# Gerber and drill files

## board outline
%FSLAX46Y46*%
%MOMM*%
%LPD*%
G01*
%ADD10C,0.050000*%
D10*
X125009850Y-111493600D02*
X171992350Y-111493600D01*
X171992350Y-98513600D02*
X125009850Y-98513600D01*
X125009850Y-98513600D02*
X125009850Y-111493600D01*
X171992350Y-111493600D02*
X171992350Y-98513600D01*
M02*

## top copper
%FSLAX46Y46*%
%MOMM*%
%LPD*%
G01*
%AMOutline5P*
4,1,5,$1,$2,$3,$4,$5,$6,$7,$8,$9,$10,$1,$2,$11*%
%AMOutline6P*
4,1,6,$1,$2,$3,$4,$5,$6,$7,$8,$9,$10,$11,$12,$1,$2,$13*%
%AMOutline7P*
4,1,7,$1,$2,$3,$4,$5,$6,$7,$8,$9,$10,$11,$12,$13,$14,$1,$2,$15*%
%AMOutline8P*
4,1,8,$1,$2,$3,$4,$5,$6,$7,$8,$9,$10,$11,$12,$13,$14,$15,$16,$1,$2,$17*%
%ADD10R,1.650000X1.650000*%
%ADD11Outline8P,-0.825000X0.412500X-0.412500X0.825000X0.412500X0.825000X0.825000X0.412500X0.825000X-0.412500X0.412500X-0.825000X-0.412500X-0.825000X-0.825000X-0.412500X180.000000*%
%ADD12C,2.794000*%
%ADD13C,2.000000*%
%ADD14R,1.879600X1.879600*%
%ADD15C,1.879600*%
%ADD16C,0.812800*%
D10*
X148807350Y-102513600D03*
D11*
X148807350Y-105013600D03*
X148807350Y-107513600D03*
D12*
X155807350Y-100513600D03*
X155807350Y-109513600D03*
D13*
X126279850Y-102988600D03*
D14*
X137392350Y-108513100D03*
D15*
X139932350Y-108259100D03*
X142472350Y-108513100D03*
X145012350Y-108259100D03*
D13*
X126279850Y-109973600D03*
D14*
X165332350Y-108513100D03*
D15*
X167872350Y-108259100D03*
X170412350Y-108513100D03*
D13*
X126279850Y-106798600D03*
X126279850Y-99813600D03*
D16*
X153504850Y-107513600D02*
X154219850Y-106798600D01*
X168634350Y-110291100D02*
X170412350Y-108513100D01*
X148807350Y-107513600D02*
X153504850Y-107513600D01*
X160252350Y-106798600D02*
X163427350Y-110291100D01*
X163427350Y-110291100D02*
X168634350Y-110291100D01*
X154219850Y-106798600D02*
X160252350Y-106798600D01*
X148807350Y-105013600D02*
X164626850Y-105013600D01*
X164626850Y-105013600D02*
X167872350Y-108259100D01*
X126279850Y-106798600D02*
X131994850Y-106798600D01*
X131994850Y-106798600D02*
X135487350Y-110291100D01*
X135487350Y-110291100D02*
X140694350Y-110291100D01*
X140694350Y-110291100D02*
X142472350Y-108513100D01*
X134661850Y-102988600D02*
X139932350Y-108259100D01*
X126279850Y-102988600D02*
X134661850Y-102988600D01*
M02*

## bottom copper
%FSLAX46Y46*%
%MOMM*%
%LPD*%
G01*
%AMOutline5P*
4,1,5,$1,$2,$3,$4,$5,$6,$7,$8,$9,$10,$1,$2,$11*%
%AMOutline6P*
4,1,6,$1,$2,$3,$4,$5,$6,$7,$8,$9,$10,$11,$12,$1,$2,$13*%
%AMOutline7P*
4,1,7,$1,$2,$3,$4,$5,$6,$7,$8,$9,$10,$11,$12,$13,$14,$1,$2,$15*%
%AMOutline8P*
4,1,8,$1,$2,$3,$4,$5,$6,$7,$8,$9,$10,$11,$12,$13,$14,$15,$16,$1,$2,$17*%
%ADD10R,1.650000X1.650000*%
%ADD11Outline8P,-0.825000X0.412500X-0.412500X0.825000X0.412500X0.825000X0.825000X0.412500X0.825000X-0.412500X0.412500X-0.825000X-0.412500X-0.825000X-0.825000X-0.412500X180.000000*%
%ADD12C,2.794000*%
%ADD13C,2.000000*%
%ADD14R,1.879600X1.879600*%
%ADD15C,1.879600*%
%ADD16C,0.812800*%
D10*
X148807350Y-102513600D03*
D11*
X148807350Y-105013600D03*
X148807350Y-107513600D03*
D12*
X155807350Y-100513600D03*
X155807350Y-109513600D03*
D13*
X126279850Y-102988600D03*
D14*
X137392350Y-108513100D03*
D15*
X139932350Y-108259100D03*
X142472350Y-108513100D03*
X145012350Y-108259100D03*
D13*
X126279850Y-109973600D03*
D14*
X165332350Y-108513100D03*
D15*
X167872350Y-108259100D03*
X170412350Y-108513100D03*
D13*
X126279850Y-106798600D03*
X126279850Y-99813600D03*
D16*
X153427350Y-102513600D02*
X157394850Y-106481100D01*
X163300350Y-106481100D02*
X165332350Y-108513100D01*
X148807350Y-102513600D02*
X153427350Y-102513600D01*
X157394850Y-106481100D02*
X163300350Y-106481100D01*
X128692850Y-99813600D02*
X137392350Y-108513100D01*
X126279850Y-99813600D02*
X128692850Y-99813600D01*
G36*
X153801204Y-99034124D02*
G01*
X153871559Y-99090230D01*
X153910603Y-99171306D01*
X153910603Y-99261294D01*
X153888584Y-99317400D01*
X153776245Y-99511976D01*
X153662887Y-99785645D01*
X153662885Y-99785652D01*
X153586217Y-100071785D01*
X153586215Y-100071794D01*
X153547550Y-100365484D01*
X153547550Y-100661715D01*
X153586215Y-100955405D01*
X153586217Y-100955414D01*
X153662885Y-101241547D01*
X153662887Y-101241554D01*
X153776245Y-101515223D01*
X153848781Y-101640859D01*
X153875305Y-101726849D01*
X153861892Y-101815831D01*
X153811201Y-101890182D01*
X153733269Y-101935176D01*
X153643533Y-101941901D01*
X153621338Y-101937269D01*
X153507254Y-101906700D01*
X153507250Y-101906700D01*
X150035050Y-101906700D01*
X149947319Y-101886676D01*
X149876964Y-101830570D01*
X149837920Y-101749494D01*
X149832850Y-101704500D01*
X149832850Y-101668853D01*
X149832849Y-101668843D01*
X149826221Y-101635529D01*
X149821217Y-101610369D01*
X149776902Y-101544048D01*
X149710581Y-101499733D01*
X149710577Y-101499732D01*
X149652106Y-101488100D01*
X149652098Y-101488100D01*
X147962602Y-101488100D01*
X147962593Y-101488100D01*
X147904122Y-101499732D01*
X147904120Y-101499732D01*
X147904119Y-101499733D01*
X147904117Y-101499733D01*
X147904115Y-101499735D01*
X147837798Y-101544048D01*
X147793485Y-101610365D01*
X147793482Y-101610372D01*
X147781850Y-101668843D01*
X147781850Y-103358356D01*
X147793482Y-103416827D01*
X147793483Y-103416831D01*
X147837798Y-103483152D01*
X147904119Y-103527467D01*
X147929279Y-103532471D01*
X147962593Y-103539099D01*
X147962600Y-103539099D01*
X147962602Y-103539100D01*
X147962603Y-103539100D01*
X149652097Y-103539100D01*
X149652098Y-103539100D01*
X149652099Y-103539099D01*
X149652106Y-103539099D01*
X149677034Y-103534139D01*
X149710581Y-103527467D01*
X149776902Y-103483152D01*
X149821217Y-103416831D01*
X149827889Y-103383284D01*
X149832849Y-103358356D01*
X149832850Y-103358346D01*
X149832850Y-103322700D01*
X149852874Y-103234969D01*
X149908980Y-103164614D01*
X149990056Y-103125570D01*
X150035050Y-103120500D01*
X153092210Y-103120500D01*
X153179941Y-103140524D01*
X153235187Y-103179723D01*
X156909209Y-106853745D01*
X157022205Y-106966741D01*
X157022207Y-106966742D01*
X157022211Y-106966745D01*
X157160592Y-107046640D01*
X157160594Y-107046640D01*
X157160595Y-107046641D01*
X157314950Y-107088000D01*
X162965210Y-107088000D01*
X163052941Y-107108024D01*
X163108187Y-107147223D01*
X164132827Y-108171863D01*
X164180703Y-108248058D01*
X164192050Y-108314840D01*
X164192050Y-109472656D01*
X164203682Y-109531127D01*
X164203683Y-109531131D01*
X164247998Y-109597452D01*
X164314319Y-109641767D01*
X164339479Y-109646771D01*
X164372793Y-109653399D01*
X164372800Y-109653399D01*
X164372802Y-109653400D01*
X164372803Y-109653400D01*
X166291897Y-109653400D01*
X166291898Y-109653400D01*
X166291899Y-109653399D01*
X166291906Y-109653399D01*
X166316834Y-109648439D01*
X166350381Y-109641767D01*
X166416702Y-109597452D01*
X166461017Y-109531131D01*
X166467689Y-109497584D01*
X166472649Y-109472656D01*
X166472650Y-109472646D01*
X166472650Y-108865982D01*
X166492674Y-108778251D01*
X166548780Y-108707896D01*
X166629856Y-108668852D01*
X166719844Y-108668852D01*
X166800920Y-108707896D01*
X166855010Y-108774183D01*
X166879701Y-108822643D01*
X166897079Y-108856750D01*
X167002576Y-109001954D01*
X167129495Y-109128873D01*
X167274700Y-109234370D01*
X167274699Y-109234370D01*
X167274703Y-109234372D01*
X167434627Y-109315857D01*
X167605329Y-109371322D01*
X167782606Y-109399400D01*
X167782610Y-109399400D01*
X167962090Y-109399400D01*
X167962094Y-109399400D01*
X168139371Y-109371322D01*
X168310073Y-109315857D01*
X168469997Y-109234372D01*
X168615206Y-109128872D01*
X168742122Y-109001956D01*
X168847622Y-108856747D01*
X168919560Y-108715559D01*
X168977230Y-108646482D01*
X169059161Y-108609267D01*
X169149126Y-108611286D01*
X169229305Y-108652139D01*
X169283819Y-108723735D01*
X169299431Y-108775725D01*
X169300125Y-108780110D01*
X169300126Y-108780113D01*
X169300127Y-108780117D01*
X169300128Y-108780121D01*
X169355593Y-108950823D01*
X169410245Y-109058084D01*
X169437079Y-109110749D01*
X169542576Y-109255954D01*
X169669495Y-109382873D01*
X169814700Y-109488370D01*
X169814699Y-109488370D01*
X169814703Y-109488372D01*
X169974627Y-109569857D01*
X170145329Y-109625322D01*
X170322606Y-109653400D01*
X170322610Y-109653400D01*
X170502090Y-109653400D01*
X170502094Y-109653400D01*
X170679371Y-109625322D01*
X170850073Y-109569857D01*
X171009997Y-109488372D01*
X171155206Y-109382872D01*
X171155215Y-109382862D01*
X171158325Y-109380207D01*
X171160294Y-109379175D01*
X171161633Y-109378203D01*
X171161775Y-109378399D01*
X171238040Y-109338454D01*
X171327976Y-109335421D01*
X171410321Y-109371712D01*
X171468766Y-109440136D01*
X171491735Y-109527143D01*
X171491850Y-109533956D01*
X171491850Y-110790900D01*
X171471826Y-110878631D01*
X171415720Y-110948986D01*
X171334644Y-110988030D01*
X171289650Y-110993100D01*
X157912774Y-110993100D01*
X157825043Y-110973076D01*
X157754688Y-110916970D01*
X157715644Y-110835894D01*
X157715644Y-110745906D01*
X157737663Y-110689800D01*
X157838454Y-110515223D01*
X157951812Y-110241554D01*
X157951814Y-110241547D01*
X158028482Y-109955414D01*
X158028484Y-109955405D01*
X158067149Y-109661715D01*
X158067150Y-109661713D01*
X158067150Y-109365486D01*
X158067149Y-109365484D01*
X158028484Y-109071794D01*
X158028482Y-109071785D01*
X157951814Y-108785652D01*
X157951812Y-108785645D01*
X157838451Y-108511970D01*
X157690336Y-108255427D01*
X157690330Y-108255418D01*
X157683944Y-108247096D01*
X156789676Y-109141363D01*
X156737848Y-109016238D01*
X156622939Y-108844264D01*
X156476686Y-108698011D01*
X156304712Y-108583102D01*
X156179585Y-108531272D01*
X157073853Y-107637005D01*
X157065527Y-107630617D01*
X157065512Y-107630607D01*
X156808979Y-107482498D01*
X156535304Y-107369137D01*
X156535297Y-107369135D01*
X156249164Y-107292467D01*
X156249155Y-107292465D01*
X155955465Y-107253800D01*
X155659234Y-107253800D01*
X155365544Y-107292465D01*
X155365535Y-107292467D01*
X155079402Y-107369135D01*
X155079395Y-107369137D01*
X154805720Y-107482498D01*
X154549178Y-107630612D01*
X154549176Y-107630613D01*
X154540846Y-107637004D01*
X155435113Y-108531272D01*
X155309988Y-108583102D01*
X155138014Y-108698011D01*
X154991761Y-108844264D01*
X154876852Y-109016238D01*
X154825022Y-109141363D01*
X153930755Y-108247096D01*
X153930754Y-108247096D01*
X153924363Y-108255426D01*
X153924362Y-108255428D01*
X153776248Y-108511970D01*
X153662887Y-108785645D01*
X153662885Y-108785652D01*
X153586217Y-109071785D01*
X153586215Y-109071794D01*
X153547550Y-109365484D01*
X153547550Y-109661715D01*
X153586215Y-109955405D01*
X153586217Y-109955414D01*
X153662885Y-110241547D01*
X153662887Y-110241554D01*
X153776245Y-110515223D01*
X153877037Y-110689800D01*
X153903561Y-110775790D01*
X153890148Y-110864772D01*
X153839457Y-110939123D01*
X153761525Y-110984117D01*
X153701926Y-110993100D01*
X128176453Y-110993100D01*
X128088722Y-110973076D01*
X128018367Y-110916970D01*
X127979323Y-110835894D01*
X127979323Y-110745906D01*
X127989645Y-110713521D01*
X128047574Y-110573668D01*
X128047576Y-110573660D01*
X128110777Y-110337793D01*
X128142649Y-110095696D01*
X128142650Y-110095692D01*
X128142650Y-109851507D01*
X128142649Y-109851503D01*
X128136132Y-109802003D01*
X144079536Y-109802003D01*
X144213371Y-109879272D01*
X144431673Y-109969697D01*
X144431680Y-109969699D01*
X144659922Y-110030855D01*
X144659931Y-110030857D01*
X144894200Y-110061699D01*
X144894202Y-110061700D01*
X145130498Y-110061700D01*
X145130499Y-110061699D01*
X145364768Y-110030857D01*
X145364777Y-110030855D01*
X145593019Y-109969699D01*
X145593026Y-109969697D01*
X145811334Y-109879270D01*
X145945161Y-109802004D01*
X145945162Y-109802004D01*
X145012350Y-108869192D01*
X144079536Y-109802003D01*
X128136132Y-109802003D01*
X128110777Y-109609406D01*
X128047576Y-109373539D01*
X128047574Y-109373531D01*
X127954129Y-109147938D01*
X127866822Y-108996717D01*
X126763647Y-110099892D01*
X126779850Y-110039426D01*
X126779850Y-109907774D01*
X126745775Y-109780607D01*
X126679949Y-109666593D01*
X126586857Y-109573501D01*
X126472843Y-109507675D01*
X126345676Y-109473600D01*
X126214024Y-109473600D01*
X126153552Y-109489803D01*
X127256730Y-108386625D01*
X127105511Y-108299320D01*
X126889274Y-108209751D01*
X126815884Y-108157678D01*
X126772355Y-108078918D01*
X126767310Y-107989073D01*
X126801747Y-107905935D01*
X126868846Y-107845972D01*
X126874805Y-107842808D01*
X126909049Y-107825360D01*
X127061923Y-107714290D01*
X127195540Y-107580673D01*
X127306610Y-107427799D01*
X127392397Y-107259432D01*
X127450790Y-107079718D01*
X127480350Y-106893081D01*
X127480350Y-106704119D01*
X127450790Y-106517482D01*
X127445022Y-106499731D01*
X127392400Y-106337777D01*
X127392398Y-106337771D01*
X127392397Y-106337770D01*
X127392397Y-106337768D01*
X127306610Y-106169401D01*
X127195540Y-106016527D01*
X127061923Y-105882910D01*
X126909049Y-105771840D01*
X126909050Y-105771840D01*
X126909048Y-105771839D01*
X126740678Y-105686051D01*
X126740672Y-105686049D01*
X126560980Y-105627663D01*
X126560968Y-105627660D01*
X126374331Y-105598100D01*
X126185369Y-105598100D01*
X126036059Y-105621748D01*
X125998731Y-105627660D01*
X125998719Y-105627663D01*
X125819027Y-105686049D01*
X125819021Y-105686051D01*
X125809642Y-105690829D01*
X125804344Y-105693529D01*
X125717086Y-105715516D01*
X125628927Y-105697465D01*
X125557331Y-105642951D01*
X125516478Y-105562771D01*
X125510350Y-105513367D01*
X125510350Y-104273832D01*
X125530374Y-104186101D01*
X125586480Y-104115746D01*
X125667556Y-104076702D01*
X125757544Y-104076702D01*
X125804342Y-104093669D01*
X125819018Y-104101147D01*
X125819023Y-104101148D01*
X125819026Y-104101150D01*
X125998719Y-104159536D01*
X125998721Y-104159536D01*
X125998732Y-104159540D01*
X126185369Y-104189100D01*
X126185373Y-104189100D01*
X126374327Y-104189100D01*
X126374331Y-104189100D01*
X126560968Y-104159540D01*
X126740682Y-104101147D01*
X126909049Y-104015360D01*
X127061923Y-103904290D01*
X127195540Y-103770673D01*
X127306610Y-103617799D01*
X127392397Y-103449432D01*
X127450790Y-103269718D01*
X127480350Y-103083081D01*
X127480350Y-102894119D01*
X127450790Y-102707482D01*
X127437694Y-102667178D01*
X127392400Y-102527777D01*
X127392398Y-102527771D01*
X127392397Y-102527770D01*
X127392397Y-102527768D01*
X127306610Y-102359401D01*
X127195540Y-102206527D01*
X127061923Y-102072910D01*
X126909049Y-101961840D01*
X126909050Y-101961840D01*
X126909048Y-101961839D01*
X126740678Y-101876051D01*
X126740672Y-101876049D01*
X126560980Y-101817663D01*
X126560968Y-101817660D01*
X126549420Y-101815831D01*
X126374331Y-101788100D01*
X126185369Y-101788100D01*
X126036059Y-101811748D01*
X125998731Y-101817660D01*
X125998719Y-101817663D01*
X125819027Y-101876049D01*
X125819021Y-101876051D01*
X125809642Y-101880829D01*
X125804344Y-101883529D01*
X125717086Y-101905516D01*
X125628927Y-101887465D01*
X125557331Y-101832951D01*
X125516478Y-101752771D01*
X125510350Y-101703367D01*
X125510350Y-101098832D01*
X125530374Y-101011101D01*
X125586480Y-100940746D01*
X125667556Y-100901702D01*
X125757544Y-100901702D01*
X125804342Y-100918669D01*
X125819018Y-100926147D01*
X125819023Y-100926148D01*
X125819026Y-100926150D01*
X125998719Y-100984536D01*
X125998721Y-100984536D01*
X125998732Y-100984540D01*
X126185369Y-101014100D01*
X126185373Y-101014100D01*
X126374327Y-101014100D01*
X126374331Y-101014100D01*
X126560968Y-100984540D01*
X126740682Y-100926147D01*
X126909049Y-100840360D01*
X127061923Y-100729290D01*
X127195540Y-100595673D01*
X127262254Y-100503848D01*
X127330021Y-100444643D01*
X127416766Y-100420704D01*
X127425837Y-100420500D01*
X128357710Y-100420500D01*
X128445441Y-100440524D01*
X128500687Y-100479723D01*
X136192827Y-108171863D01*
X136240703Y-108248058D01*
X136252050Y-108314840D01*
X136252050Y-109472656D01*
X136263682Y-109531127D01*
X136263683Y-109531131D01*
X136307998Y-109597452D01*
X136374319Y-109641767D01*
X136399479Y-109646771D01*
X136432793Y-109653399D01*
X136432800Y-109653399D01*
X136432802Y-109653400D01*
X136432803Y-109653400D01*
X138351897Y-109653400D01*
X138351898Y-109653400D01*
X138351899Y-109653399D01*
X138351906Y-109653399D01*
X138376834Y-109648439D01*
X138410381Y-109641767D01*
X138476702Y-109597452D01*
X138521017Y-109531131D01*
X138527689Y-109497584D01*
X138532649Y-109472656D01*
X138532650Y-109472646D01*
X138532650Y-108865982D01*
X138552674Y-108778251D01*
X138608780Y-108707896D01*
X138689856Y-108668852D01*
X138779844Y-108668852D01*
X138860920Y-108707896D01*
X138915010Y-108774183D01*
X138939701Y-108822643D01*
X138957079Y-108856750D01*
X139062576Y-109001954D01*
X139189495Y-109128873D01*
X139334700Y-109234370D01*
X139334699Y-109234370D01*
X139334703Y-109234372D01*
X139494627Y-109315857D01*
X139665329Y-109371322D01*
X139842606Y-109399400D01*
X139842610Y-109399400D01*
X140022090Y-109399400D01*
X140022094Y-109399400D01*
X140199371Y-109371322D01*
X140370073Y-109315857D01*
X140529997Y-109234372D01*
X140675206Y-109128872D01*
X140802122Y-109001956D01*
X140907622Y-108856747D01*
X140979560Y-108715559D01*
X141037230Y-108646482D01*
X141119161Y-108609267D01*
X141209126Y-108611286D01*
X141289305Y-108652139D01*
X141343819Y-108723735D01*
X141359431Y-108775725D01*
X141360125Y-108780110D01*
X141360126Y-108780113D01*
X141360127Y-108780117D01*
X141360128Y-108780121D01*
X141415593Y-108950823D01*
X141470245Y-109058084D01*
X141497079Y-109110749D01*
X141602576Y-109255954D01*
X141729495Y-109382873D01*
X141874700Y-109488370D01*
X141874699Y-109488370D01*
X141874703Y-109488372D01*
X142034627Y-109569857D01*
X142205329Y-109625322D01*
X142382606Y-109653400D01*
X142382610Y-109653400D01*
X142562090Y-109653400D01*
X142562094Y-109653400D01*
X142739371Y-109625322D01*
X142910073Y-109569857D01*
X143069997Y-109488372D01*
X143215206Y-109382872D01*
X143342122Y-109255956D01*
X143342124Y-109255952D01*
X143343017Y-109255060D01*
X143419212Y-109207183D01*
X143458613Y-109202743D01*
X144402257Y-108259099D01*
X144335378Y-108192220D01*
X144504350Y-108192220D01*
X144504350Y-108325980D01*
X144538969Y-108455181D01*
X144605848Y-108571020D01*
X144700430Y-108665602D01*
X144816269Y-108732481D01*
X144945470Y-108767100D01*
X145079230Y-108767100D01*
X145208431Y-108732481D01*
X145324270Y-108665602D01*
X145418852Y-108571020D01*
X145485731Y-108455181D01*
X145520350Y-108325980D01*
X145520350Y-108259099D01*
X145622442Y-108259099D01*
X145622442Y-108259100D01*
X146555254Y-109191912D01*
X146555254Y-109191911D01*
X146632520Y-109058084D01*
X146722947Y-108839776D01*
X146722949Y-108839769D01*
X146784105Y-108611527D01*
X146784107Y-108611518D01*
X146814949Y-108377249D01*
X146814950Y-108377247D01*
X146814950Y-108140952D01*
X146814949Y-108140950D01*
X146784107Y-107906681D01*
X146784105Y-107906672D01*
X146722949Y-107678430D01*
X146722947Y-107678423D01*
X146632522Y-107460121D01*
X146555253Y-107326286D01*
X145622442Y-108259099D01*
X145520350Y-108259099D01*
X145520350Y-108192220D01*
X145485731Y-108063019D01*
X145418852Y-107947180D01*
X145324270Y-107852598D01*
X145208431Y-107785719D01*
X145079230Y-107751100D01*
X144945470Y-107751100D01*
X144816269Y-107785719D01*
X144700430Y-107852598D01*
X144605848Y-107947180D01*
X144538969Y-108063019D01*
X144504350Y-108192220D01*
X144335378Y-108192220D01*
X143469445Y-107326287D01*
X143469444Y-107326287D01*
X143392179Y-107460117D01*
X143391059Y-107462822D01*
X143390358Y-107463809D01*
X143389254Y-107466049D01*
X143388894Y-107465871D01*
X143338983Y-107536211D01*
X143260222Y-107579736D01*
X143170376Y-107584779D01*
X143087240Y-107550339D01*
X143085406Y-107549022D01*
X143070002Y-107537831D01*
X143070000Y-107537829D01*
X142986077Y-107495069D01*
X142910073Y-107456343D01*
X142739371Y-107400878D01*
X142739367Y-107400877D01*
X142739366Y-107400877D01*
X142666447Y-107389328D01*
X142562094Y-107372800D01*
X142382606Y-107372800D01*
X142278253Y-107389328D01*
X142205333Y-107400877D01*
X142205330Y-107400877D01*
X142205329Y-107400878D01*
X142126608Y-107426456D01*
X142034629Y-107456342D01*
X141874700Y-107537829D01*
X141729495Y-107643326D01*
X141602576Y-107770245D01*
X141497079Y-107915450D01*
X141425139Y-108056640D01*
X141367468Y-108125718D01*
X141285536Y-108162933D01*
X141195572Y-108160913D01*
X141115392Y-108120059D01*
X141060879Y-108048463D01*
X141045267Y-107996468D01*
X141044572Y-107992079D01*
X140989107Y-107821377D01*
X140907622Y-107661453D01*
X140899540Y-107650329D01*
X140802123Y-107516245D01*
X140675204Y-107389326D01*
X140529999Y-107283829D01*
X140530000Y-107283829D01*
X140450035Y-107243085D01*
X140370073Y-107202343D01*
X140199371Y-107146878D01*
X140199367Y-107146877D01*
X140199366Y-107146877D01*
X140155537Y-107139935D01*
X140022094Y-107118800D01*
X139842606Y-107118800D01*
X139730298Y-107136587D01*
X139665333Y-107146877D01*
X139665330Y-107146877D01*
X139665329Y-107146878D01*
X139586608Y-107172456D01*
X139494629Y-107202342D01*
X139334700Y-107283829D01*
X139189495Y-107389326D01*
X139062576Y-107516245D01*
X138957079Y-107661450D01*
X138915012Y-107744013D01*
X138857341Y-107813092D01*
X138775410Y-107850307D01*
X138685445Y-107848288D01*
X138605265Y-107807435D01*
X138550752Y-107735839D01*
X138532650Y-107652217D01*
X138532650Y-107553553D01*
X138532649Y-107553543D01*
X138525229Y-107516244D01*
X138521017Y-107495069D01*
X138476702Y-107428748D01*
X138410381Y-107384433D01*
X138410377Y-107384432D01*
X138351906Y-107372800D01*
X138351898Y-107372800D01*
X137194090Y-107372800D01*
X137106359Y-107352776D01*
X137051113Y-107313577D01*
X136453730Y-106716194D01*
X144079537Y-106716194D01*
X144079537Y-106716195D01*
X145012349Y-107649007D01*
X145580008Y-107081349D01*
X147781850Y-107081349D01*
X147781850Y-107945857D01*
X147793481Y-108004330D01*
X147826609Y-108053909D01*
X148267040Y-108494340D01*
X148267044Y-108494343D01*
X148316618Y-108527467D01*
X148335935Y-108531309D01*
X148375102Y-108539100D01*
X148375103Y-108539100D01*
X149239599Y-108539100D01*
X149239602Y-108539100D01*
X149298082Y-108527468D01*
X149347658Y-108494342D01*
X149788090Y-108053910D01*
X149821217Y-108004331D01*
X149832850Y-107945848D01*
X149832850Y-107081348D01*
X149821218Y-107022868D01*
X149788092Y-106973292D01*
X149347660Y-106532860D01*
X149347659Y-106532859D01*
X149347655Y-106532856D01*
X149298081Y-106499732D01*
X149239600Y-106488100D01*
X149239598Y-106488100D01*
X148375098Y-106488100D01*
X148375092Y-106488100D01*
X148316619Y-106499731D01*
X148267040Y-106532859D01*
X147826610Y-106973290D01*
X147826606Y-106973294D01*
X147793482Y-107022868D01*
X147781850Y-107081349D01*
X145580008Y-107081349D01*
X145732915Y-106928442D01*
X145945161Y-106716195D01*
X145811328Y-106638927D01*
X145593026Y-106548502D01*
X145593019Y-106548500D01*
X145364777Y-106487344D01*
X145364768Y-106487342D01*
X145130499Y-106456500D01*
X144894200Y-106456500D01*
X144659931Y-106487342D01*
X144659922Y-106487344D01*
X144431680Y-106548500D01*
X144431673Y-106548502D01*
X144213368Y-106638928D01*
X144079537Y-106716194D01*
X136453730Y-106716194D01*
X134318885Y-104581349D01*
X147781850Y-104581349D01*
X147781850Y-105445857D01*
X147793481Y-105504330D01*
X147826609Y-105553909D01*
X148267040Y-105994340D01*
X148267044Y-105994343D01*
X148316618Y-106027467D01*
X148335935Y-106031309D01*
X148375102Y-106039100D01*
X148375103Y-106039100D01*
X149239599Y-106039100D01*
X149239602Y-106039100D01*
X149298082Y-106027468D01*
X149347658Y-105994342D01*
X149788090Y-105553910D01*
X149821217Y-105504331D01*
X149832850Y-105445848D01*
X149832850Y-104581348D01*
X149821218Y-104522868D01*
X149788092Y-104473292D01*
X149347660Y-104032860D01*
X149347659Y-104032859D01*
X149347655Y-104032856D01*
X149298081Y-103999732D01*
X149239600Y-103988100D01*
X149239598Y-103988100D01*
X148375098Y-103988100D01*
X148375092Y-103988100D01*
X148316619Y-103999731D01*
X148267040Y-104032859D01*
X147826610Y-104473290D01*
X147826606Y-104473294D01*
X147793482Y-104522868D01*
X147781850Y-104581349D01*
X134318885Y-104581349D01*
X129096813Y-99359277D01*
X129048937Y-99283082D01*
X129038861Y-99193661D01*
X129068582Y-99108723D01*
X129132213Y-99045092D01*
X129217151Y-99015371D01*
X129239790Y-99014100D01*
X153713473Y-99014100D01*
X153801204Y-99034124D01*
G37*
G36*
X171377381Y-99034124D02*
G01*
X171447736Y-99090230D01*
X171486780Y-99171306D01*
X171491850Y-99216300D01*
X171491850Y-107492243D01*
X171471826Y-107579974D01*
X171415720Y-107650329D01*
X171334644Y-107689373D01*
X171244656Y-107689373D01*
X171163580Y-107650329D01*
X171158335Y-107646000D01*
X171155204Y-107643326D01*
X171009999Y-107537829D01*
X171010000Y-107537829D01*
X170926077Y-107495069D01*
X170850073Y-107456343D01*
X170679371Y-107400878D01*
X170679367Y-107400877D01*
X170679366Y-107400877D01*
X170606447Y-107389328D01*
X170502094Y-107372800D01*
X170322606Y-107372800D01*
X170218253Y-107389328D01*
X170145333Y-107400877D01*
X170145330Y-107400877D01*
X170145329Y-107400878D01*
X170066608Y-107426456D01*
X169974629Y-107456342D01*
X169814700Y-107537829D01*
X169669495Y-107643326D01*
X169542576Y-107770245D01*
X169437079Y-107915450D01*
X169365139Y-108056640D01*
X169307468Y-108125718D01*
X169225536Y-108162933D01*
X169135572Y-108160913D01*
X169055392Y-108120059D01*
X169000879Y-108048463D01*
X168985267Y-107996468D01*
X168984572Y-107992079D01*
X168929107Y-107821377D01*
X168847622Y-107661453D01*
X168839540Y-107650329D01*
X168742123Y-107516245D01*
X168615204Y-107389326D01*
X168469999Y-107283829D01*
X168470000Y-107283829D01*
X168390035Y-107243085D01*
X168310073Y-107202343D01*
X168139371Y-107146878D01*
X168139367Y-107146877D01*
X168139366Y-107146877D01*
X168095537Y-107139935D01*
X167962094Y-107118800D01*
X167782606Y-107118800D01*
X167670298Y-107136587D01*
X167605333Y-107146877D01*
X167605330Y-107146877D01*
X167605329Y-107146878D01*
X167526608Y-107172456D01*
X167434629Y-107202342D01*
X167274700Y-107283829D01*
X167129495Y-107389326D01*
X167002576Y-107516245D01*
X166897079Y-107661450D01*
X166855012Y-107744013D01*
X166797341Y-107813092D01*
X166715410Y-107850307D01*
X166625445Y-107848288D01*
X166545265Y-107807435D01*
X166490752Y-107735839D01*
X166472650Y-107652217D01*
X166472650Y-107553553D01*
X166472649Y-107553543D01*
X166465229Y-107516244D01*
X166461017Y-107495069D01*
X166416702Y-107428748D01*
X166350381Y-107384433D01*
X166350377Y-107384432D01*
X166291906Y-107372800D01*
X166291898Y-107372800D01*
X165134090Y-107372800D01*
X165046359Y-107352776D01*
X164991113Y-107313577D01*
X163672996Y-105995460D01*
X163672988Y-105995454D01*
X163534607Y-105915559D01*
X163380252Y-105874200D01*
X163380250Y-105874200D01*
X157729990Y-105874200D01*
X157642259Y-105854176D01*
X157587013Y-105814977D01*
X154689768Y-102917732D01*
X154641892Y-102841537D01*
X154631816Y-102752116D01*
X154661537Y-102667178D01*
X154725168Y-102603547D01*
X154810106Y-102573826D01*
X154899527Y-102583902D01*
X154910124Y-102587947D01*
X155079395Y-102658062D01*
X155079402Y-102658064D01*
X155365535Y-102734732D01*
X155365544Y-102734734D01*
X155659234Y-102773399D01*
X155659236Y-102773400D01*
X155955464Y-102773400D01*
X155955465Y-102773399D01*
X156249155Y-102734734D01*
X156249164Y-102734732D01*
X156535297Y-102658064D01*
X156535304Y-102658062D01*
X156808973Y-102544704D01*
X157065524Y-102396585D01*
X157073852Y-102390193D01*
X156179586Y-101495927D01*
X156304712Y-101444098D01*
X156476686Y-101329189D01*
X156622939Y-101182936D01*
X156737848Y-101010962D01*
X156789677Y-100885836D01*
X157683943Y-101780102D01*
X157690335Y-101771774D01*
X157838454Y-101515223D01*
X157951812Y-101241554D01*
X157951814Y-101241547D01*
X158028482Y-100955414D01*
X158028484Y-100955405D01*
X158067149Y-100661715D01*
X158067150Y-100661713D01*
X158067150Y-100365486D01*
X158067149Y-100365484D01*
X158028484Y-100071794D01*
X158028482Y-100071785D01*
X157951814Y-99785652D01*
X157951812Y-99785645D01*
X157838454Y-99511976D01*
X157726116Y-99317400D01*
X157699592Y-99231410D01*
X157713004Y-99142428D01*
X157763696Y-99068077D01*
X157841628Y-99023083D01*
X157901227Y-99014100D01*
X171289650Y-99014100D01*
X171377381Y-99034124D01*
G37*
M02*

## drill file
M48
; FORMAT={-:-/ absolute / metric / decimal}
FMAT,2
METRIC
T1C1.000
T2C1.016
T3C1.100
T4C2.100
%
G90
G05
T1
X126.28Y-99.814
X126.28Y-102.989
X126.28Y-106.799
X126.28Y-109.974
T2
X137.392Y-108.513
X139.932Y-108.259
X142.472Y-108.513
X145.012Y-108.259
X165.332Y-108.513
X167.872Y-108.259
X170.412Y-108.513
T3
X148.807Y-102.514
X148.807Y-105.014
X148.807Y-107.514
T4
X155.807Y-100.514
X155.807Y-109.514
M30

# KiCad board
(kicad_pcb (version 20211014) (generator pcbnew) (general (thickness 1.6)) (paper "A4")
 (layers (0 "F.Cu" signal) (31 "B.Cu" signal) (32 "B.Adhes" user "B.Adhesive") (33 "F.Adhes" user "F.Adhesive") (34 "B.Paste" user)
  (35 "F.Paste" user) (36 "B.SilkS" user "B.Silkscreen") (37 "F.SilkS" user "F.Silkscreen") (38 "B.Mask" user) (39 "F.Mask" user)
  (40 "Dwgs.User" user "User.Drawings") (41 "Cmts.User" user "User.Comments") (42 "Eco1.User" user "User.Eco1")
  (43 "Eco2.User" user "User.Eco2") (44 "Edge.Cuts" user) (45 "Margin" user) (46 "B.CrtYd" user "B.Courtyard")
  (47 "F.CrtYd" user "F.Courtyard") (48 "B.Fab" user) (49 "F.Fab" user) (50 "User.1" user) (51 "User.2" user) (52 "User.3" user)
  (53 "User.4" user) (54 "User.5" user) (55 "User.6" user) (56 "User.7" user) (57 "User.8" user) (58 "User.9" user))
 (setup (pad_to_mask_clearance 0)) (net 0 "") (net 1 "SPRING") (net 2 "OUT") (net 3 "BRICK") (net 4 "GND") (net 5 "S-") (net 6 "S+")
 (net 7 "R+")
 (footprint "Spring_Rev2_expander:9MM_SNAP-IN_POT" (layer "F.Cu") (at 155.80735 105.0136 -90)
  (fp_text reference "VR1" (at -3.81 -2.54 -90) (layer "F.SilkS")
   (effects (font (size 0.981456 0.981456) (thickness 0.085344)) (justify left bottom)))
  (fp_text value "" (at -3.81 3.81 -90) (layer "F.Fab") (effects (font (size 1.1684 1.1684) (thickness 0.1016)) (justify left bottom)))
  (pad "1" thru_hole rect (at -2.5 7 180) (size 1.65 1.65) (drill 1.1) (layers *.Cu *.Mask) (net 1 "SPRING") (solder_mask_margin 0.0635))
  (pad "2" thru_hole roundrect (at 0 7 180) (size 1.65 1.65) (drill 1.1) (layers *.Cu *.Mask) (roundrect_rratio 0.25) (chamfer_ratio 0.25)
   (chamfer top_left top_right bottom_left bottom_right) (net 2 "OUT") (solder_mask_margin 0.0635))
  (pad "3" thru_hole roundrect (at 2.5 7 180) (size 1.65 1.65) (drill 1.1) (layers *.Cu *.Mask) (roundrect_rratio 0.25) (chamfer_ratio 0.25)
   (chamfer top_left top_right bottom_left bottom_right) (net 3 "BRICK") (solder_mask_margin 0.0635))
  (pad "CHASSIS1" thru_hole circle (at -4.5 0 180) (size 2.794 2.794) (drill 2.1) (layers *.Cu *.Mask) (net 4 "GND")
   (solder_mask_margin 0.0635))
  (pad "CHASSIS2" thru_hole circle (at 4.5 0 180) (size 2.794 2.794) (drill 2.1) (layers *.Cu *.Mask) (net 4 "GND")
   (solder_mask_margin 0.0635)))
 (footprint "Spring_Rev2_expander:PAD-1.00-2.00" (layer "B.Cu") (at 126.27985 102.9886 180)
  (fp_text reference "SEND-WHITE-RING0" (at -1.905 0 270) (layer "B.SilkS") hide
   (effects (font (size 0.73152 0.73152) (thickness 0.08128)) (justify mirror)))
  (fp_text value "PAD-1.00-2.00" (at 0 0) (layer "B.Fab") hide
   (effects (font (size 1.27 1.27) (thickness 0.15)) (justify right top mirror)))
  (pad "1" thru_hole circle (at 0 0 180) (size 2 2) (drill 1) (layers *.Cu *.Mask) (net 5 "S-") (solder_mask_margin 0.0635)))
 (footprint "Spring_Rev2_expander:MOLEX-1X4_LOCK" (layer "B.Cu") (at 137.39235 108.3861)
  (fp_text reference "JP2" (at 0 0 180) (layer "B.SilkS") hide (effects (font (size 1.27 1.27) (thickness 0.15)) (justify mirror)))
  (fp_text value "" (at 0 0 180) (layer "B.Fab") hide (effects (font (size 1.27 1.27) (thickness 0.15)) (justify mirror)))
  (pad "1" thru_hole rect (at 0 0.127) (size 1.8796 1.8796) (drill 1.016) (layers *.Cu *.Mask) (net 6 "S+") (solder_mask_margin 0.0635))
  (pad "2" thru_hole circle (at 2.54 -0.127) (size 1.8796 1.8796) (drill 1.016) (layers *.Cu *.Mask) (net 5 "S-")
   (solder_mask_margin 0.0635))
  (pad "3" thru_hole circle (at 5.08 0.127) (size 1.8796 1.8796) (drill 1.016) (layers *.Cu *.Mask) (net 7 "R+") (solder_mask_margin 0.0635))
  (pad "4" thru_hole circle (at 7.62 -0.127) (size 1.8796 1.8796) (drill 1.016) (layers *.Cu *.Mask) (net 4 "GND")
   (solder_mask_margin 0.0635)))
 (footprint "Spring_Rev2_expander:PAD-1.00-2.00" (layer "B.Cu") (at 126.27985 109.9736 180)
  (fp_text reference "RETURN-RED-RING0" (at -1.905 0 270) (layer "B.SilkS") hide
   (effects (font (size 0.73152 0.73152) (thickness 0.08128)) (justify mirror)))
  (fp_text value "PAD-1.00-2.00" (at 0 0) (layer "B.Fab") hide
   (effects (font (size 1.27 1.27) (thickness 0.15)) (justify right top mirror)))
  (pad "1" thru_hole circle (at 0 0 180) (size 2 2) (drill 1) (layers *.Cu *.Mask) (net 4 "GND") (solder_mask_margin 0.0635)))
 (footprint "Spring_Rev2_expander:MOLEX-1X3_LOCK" (layer "B.Cu") (at 165.33235 108.3861)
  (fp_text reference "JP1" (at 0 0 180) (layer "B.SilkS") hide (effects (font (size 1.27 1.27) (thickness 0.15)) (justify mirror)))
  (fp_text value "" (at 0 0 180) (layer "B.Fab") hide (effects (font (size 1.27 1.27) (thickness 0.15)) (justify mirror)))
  (pad "1" thru_hole rect (at 0 0.127) (size 1.8796 1.8796) (drill 1.016) (layers *.Cu *.Mask) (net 1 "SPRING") (solder_mask_margin 0.0635))
  (pad "2" thru_hole circle (at 2.54 -0.127) (size 1.8796 1.8796) (drill 1.016) (layers *.Cu *.Mask) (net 2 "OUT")
   (solder_mask_margin 0.0635))
  (pad "3" thru_hole circle (at 5.08 0.127) (size 1.8796 1.8796) (drill 1.016) (layers *.Cu *.Mask) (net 3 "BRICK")
   (solder_mask_margin 0.0635)))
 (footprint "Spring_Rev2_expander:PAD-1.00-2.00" (layer "B.Cu") (at 126.27985 106.7986 180)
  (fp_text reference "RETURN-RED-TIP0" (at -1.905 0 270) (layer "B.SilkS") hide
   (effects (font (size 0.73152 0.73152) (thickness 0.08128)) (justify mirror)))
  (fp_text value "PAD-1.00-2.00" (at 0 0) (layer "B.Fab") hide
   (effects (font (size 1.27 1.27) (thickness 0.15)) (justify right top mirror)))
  (pad "1" thru_hole circle (at 0 0 180) (size 2 2) (drill 1) (layers *.Cu *.Mask) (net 7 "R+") (solder_mask_margin 0.0635)))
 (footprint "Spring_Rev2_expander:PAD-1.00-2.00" (layer "B.Cu") (at 126.27985 99.8136 180)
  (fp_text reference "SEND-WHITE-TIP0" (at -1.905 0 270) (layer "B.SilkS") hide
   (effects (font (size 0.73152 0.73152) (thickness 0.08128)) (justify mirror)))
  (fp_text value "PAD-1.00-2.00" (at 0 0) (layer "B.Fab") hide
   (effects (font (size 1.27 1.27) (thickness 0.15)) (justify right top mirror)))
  (pad "1" thru_hole circle (at 0 0 180) (size 2 2) (drill 1) (layers *.Cu *.Mask) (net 6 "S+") (solder_mask_margin 0.0635)))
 (gr_line (start 125.00985 111.4936) (end 171.99235 111.4936) (layer "Edge.Cuts") (width 0.05))
 (gr_line (start 171.99235 98.5136) (end 125.00985 98.5136) (layer "Edge.Cuts") (width 0.05))
 (gr_line (start 125.00985 98.5136) (end 125.00985 111.4936) (layer "Edge.Cuts") (width 0.05))
 (gr_line (start 171.99235 111.4936) (end 171.99235 98.5136) (layer "Edge.Cuts") (width 0.05))
 (segment (start 153.50485 107.5136) (end 154.21985 106.7986) (width 0.8128) (layer "F.Cu") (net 3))
 (segment (start 168.63435 110.2911) (end 170.41235 108.5131) (width 0.8128) (layer "F.Cu") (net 3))
 (segment (start 148.80735 107.5136) (end 153.50485 107.5136) (width 0.8128) (layer "F.Cu") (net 3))
 (segment (start 160.25235 106.7986) (end 163.42735 110.2911) (width 0.8128) (layer "F.Cu") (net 3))
 (segment (start 163.42735 110.2911) (end 168.63435 110.2911) (width 0.8128) (layer "F.Cu") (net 3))
 (segment (start 154.21985 106.7986) (end 160.25235 106.7986) (width 0.8128) (layer "F.Cu") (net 3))
 (segment (start 148.80735 105.0136) (end 164.62685 105.0136) (width 0.8128) (layer "F.Cu") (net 2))
 (segment (start 164.62685 105.0136) (end 167.87235 108.2591) (width 0.8128) (layer "F.Cu") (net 2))
 (segment (start 153.42735 102.5136) (end 157.39485 106.4811) (width 0.8128) (layer "B.Cu") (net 1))
 (segment (start 163.30035 106.4811) (end 165.33235 108.5131) (width 0.8128) (layer "B.Cu") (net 1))
 (segment (start 148.80735 102.5136) (end 153.42735 102.5136) (width 0.8128) (layer "B.Cu") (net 1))
 (segment (start 157.39485 106.4811) (end 163.30035 106.4811) (width 0.8128) (layer "B.Cu") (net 1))
 (segment (start 126.27985 106.7986) (end 131.99485 106.7986) (width 0.8128) (layer "F.Cu") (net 7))
 (segment (start 131.99485 106.7986) (end 135.48735 110.2911) (width 0.8128) (layer "F.Cu") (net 7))
 (segment (start 135.48735 110.2911) (end 140.69435 110.2911) (width 0.8128) (layer "F.Cu") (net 7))
 (segment (start 140.69435 110.2911) (end 142.47235 108.5131) (width 0.8128) (layer "F.Cu") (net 7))
 (segment (start 134.66185 102.9886) (end 139.93235 108.2591) (width 0.8128) (layer "F.Cu") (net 5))
 (segment (start 126.27985 102.9886) (end 134.66185 102.9886) (width 0.8128) (layer "F.Cu") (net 5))
 (segment (start 128.69285 99.8136) (end 137.39235 108.5131) (width 0.8128) (layer "B.Cu") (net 6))
 (segment (start 126.27985 99.8136) (end 128.69285 99.8136) (width 0.8128) (layer "B.Cu") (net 6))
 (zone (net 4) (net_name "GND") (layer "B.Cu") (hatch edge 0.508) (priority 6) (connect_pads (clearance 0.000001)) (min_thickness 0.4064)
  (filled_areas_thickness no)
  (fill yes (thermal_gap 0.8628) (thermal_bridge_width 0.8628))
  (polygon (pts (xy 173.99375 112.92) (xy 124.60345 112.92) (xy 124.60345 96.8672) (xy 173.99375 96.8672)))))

